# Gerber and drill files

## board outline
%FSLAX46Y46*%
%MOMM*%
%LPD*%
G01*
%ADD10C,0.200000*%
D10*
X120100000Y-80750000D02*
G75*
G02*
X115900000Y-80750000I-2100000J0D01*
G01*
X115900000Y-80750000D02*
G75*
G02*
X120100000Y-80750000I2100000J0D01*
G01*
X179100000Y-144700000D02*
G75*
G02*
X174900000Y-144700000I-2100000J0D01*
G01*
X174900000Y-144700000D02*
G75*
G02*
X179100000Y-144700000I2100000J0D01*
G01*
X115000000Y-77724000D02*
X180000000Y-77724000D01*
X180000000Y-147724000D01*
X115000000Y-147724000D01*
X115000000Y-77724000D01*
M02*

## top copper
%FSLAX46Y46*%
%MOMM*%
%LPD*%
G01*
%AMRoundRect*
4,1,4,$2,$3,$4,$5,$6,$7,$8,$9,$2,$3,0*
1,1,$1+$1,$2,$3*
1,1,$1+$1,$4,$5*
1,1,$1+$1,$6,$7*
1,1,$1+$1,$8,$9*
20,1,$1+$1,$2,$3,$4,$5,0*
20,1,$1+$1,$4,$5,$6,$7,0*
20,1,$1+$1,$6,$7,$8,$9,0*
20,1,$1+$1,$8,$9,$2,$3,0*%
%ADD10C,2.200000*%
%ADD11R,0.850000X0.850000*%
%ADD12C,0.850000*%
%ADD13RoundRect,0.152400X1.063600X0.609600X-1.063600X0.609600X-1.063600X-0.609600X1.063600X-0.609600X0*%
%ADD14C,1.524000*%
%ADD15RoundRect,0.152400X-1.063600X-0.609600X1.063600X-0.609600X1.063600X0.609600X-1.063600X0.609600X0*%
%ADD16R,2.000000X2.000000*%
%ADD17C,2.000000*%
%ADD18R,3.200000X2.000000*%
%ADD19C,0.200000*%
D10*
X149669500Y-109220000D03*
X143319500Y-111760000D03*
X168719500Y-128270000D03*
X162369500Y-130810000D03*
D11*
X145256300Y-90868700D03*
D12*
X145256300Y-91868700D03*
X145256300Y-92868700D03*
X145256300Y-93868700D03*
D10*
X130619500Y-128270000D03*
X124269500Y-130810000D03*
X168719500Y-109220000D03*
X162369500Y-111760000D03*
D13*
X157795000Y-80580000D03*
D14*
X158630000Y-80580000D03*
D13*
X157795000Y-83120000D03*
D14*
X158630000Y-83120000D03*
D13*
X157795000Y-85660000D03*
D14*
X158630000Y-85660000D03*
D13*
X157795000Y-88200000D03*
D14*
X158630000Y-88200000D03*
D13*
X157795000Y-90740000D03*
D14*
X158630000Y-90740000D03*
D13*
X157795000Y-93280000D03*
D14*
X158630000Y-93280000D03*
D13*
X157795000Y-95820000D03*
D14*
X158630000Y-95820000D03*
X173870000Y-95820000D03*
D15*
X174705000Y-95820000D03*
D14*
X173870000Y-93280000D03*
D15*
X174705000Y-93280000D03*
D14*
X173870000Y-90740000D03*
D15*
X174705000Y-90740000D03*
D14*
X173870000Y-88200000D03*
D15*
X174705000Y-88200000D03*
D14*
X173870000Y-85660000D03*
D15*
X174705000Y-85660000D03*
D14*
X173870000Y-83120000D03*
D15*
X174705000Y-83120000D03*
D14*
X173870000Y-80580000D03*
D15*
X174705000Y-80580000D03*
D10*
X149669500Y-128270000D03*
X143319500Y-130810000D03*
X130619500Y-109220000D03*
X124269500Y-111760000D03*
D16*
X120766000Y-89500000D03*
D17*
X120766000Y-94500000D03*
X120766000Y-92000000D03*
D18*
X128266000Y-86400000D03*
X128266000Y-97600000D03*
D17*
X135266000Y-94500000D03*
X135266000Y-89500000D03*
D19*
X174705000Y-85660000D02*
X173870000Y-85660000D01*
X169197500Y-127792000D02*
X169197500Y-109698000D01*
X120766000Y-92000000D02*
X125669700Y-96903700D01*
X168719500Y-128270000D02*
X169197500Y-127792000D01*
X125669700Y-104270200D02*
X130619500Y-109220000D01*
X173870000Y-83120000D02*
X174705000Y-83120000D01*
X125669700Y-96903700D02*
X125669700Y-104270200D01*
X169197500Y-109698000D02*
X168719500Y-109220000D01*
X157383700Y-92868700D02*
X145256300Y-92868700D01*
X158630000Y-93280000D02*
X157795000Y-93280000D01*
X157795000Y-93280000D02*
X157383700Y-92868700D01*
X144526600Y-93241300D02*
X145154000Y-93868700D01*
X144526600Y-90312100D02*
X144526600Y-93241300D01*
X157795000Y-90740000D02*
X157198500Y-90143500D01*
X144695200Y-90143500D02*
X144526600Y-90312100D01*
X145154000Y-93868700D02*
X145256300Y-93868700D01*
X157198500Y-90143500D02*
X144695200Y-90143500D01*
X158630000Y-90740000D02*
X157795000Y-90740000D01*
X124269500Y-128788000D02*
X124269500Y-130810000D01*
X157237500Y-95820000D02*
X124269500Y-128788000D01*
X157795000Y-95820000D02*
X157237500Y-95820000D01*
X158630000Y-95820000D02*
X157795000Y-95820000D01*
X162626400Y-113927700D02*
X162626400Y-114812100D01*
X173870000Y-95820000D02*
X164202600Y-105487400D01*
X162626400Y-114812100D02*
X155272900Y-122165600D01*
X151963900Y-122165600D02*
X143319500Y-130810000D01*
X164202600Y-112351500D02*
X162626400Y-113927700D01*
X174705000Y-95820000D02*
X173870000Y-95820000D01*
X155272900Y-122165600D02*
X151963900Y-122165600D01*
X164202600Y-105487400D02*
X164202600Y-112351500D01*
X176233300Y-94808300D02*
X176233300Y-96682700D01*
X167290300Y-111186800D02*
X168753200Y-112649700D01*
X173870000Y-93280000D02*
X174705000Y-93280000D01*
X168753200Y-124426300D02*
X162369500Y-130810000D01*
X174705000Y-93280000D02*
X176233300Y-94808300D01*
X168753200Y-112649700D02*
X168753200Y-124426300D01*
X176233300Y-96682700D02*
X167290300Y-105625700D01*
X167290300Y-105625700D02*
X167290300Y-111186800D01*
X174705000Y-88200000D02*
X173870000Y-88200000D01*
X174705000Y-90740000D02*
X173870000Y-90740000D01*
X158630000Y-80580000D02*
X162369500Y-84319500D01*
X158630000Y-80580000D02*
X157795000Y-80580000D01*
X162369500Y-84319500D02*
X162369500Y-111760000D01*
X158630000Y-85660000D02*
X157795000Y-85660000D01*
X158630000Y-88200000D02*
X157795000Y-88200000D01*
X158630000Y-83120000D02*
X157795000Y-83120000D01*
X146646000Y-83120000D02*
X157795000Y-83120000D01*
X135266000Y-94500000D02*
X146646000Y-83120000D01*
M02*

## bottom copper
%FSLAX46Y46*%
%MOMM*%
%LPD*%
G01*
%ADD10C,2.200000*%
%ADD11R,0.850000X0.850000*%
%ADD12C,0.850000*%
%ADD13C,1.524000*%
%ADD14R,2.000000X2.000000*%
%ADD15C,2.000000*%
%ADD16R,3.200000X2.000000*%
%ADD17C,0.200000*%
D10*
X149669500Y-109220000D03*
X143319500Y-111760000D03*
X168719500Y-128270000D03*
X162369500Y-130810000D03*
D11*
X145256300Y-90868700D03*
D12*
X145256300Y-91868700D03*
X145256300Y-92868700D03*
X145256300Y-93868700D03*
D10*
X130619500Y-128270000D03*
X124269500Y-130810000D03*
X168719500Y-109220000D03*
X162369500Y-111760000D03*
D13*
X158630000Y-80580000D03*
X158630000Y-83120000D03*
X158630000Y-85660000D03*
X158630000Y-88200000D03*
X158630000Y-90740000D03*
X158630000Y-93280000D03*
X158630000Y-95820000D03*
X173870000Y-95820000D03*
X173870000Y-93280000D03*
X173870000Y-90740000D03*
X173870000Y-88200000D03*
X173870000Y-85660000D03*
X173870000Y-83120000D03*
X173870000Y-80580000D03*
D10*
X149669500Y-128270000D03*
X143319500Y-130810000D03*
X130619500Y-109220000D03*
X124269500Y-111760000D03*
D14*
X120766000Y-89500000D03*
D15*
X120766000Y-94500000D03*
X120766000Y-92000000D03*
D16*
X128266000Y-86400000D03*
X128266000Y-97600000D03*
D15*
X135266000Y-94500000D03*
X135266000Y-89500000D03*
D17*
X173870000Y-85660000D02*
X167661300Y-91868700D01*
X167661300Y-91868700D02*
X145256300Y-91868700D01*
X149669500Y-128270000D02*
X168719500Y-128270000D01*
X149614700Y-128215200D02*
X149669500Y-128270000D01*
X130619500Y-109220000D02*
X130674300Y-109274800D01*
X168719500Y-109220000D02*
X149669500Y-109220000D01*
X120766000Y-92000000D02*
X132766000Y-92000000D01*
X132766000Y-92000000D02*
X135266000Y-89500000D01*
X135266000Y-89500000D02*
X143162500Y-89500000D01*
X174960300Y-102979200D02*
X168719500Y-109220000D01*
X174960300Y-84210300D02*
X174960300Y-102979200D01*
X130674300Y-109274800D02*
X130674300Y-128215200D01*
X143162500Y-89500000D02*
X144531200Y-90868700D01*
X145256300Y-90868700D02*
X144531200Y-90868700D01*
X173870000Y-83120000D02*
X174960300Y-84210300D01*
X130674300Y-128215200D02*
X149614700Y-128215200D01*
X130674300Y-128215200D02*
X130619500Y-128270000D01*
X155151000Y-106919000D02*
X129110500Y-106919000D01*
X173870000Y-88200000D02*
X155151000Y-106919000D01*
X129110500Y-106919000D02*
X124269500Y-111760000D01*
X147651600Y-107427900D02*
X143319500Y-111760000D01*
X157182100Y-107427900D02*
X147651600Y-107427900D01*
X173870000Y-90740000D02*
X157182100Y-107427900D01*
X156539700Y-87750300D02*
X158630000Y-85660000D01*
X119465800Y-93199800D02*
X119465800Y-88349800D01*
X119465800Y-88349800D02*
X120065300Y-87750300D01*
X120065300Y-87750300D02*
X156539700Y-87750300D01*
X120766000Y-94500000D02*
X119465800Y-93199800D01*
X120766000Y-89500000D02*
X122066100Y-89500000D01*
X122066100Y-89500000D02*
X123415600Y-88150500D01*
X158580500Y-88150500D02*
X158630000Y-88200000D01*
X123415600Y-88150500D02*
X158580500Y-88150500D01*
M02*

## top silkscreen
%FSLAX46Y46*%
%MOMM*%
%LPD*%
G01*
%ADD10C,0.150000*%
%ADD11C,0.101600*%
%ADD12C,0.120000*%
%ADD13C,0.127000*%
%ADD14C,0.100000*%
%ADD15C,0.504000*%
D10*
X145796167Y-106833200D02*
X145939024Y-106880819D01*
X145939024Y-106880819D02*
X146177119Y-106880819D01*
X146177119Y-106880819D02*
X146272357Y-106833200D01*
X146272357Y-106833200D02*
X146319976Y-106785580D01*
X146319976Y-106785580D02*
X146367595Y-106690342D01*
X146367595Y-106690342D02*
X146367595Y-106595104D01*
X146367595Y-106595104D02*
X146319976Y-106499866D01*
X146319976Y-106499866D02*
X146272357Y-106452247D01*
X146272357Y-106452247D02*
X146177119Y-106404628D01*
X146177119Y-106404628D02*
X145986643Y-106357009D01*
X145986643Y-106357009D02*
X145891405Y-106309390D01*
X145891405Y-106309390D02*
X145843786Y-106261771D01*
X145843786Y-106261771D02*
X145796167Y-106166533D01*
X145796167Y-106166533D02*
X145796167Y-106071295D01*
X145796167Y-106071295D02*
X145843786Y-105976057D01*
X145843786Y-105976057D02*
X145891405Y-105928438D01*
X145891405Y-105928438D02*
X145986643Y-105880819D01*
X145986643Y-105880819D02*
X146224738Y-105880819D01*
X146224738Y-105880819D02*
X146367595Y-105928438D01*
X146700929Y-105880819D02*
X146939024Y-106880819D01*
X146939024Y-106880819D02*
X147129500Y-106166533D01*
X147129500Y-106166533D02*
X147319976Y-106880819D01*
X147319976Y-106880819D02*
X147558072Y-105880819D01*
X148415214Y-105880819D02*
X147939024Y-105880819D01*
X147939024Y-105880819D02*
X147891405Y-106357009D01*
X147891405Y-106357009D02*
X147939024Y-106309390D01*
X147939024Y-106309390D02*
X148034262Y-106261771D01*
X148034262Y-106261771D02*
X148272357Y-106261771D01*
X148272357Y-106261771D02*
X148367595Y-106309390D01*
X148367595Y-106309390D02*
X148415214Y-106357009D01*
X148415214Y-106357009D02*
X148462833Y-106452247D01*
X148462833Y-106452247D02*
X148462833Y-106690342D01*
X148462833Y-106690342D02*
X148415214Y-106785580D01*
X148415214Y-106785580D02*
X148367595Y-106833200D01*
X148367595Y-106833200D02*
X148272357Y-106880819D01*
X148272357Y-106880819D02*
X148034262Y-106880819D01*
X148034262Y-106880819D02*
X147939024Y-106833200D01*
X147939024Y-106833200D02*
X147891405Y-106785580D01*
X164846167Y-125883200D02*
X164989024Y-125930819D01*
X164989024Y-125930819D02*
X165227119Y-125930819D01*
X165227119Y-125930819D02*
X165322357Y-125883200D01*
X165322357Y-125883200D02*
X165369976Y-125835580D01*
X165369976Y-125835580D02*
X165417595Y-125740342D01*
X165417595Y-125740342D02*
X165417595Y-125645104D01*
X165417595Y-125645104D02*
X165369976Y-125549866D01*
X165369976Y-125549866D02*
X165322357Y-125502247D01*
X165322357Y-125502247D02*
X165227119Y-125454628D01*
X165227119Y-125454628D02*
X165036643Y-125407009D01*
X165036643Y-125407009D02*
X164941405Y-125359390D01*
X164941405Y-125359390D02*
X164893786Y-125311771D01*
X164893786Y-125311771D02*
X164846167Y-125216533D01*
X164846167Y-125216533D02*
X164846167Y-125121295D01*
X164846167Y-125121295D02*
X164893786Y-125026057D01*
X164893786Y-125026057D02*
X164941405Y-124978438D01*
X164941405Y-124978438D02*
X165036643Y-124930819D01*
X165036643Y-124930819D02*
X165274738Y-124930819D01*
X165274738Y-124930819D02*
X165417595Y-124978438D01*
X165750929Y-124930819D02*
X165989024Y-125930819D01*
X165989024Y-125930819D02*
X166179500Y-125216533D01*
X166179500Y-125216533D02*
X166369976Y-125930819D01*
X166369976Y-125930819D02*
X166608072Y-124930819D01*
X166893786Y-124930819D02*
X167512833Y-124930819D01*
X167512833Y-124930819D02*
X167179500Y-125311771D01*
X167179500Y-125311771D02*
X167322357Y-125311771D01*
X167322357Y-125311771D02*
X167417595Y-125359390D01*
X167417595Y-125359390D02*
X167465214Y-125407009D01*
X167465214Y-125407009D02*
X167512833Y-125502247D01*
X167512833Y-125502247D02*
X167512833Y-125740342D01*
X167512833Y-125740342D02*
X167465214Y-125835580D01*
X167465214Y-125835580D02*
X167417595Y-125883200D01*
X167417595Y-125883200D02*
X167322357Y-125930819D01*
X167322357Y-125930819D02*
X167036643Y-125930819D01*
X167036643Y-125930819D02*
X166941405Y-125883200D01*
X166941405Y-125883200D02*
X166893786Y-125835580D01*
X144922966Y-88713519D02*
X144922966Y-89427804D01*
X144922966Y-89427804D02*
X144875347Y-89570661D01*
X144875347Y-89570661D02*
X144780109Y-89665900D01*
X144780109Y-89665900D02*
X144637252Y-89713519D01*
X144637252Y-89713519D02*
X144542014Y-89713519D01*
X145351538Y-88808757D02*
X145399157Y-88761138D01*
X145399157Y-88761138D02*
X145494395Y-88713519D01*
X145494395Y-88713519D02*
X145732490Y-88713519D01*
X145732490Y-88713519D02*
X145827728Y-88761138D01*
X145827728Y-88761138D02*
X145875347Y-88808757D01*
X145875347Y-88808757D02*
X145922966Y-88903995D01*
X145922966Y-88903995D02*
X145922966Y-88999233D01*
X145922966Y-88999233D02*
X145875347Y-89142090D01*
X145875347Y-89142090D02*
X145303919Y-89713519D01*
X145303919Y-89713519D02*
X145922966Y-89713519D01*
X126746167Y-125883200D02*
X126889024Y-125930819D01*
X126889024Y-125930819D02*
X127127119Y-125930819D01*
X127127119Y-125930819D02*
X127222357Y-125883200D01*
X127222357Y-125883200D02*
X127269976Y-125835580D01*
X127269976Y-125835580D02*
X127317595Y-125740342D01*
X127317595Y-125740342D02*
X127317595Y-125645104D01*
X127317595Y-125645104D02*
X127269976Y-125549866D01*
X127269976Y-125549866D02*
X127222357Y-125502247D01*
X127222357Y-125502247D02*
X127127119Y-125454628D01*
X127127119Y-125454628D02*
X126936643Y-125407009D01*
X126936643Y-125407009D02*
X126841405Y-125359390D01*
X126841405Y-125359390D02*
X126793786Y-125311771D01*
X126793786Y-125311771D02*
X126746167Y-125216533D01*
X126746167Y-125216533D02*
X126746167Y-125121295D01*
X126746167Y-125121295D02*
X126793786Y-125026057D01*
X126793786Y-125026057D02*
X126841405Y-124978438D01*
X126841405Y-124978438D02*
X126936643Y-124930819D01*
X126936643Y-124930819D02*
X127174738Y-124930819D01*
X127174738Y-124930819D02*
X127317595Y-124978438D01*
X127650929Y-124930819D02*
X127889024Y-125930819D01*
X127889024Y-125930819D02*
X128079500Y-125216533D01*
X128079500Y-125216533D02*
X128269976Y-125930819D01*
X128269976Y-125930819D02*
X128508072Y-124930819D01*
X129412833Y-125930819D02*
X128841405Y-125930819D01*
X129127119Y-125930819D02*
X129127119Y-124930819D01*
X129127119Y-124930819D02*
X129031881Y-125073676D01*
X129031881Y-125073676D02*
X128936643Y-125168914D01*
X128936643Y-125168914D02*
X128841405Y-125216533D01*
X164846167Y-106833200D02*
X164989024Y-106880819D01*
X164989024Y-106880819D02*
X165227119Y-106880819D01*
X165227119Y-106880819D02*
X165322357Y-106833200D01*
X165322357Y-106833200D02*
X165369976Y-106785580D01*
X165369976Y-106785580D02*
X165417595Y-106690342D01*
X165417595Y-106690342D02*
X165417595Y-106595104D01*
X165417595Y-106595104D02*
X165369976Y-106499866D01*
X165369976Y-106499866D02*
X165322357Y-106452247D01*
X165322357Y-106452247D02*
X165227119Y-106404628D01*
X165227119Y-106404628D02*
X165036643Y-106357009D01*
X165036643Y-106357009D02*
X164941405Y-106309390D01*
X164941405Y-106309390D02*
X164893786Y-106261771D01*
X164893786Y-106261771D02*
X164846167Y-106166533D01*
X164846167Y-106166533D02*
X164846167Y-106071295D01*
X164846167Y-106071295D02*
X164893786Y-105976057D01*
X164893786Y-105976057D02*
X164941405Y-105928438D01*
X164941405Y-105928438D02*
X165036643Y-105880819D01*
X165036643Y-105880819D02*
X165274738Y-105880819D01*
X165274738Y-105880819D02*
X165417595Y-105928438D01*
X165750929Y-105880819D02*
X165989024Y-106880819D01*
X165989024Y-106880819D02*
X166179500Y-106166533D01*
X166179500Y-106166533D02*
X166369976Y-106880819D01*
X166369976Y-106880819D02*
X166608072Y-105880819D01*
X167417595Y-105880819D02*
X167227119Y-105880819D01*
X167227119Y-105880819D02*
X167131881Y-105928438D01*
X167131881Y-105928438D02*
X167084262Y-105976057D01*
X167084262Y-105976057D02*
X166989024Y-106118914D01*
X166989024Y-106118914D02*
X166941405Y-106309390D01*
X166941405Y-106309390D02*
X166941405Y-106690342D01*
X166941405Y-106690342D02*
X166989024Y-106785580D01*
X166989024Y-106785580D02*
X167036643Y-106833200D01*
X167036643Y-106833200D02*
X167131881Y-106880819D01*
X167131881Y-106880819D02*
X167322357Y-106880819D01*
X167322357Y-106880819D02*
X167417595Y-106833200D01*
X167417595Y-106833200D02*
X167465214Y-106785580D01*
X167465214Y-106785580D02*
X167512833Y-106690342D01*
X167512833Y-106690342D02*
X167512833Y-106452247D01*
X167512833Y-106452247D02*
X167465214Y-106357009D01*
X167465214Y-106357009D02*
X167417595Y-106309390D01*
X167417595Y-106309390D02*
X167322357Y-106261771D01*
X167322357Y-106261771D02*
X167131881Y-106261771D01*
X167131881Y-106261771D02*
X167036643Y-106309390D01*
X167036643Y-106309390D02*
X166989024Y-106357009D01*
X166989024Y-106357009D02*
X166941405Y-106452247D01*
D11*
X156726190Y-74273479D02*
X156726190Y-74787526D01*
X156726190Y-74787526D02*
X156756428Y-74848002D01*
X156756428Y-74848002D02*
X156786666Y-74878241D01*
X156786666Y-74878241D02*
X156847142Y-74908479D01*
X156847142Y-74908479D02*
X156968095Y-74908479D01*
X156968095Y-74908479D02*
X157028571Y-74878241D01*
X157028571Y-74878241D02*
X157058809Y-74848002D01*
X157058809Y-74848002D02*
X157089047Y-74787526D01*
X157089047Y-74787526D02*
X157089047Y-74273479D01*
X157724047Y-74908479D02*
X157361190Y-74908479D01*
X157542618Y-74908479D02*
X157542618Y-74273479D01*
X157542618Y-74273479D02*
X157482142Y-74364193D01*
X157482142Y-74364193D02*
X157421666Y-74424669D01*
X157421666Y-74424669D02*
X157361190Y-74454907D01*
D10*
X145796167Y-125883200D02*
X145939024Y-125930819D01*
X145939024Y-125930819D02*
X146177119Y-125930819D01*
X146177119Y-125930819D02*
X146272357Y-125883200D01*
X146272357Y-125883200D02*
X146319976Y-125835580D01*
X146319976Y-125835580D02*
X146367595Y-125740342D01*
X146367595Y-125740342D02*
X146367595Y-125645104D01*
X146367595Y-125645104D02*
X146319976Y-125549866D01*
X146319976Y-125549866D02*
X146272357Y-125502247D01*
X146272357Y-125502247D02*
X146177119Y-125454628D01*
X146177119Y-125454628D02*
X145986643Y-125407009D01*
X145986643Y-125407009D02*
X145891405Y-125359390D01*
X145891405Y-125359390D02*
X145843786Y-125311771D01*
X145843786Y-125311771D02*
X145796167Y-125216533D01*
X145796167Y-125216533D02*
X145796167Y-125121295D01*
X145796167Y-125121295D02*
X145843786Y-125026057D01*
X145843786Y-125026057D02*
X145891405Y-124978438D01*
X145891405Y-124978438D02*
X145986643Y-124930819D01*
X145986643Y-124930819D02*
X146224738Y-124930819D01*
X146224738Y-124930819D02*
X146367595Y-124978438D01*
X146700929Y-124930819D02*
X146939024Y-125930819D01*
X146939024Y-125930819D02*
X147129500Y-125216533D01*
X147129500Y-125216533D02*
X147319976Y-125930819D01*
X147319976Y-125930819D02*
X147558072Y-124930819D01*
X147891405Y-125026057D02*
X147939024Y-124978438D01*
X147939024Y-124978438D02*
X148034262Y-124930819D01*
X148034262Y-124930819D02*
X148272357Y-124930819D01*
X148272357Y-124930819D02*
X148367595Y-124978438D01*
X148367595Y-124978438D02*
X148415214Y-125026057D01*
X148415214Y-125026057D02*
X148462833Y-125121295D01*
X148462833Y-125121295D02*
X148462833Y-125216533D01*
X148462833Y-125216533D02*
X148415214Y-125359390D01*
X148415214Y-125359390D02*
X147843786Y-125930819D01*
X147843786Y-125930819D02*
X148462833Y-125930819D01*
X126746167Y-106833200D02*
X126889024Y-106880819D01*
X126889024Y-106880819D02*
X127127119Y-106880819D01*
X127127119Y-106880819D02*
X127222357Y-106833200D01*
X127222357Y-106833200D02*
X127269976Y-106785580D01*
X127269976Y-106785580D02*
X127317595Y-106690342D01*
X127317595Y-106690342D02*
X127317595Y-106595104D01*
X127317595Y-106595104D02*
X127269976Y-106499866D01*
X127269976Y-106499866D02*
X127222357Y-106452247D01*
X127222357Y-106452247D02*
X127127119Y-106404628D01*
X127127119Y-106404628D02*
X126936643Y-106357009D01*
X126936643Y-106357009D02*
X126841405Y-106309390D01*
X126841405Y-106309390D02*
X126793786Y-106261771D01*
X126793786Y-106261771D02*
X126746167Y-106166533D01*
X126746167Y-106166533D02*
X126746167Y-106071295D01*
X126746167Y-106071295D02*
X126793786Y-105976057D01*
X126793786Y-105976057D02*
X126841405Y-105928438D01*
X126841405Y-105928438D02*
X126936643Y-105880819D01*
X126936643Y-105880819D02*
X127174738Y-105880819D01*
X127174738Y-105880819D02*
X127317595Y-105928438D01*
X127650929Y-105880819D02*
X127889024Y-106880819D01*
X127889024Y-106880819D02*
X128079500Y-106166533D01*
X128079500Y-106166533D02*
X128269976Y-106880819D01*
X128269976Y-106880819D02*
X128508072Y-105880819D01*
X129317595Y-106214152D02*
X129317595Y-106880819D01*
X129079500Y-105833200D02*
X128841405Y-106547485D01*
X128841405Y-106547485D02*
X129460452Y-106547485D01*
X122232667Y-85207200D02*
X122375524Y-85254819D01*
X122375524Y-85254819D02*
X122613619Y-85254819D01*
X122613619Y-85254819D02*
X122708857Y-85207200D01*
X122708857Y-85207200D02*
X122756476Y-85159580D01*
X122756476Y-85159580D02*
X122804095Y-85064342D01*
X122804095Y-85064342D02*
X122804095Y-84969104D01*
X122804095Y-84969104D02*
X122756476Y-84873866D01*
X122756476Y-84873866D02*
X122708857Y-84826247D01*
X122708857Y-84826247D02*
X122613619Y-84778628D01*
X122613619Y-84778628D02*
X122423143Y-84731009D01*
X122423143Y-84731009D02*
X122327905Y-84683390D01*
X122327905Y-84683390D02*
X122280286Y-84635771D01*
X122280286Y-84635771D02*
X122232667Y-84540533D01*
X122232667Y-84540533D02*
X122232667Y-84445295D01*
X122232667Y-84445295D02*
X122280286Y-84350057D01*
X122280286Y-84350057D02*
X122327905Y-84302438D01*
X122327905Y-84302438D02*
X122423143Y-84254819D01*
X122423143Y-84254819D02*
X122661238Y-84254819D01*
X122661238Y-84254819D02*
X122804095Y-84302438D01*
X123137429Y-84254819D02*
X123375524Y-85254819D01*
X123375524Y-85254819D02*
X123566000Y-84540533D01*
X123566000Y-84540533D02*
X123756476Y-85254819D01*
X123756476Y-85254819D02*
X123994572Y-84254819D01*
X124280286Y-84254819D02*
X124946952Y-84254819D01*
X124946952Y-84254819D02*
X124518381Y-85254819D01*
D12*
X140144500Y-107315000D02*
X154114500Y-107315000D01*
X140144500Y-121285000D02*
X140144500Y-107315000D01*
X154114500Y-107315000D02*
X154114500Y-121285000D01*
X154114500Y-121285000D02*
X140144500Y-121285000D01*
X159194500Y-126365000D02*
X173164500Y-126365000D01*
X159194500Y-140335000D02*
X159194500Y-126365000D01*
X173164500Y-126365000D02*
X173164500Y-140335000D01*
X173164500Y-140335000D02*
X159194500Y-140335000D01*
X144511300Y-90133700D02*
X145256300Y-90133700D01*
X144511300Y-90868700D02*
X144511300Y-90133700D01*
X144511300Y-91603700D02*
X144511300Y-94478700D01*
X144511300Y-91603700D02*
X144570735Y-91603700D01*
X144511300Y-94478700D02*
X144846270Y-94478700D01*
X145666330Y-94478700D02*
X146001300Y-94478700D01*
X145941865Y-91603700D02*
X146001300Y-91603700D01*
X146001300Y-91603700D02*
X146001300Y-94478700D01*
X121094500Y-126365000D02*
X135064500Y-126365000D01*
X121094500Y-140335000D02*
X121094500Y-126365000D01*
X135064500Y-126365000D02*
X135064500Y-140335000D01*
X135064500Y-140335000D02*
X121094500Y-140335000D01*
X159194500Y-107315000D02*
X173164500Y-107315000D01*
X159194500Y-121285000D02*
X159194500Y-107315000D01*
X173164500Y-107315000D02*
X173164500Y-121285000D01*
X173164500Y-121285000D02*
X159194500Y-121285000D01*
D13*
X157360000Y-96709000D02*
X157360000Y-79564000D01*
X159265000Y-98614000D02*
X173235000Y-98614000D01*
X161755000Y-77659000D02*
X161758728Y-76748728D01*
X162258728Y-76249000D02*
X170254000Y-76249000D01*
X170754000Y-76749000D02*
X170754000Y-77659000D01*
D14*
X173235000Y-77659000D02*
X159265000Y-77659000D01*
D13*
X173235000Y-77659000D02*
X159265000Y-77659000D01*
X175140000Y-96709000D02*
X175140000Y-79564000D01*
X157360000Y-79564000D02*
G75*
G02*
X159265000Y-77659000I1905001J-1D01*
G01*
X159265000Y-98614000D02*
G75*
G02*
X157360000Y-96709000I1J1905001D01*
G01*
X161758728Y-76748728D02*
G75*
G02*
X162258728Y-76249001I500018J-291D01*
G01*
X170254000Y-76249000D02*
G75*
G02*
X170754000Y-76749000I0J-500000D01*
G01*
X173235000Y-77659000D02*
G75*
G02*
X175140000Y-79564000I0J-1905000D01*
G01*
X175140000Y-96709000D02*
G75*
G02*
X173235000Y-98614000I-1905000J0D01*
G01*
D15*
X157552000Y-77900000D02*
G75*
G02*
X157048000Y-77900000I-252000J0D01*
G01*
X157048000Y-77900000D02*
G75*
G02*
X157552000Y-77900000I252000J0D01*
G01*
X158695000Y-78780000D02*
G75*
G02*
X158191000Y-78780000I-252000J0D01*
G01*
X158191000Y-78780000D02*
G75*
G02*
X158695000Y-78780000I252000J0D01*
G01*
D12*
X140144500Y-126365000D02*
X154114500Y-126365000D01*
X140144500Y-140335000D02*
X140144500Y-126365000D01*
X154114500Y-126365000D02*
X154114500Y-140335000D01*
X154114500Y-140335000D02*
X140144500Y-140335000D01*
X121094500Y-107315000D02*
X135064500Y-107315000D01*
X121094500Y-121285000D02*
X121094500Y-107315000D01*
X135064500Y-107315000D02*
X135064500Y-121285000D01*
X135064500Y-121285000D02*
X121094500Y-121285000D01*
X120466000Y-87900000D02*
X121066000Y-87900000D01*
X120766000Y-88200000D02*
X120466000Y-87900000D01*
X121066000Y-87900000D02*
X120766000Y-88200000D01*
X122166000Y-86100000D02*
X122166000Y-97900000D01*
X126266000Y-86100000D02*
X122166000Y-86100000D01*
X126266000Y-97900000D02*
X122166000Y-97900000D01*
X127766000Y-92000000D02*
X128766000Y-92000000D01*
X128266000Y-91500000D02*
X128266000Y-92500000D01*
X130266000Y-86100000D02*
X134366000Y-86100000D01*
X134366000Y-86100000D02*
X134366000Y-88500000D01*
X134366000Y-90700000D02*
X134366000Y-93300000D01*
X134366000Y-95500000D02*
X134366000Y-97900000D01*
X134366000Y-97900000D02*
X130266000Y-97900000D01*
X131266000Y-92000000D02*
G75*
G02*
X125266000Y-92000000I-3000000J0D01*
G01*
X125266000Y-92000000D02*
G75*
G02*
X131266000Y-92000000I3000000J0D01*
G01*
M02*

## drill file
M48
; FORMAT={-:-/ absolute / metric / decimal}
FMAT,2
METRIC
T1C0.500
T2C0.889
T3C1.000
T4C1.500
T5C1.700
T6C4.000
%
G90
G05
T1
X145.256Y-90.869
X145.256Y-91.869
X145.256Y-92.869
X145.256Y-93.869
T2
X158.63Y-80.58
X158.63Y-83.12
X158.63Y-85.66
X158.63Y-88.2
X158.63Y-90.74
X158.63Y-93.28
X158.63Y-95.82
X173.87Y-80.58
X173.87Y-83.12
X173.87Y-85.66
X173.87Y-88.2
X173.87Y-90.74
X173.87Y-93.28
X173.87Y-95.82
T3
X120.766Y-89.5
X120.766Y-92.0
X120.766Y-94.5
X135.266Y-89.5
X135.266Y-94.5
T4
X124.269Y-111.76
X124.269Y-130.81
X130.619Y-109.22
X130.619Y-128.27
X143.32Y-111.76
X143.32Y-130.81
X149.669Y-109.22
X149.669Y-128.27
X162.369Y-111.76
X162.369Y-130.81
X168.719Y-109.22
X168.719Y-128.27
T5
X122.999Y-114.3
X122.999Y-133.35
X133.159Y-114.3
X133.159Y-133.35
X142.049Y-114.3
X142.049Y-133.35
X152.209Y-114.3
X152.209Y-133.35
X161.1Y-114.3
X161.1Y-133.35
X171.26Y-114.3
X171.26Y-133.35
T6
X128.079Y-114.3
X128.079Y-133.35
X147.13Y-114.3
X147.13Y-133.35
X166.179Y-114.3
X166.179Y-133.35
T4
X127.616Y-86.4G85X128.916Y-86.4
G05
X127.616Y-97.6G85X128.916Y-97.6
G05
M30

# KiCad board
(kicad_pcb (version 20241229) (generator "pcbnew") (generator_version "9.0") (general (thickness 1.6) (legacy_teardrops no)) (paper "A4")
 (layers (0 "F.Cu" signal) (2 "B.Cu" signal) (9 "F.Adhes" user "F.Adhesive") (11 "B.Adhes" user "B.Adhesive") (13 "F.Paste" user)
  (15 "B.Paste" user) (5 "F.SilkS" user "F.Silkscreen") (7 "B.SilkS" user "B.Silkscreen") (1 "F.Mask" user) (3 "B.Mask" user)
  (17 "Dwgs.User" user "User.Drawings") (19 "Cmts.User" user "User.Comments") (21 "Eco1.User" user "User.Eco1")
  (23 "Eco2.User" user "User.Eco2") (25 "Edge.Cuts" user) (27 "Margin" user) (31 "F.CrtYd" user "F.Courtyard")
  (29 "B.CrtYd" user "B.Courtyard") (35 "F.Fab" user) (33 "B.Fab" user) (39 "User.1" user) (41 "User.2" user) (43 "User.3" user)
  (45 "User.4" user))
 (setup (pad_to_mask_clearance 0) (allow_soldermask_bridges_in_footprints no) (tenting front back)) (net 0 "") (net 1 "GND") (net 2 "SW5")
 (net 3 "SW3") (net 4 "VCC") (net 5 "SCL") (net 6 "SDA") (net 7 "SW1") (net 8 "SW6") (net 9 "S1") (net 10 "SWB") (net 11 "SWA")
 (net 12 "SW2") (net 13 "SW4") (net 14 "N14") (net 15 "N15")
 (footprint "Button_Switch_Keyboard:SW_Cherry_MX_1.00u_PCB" (layer "F.Cu") (at 149.6695 109.22)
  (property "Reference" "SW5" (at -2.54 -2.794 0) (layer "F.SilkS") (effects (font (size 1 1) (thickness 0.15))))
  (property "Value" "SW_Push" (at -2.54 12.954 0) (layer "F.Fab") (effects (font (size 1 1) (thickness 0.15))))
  (fp_line (start -9.525 -1.905) (end 4.445 -1.905) (stroke (width 0.12) (type solid)) (layer "F.SilkS"))
  (fp_line (start -9.525 12.065) (end -9.525 -1.905) (stroke (width 0.12) (type solid)) (layer "F.SilkS"))
  (fp_line (start 4.445 -1.905) (end 4.445 12.065) (stroke (width 0.12) (type solid)) (layer "F.SilkS"))
  (fp_line (start 4.445 12.065) (end -9.525 12.065) (stroke (width 0.12) (type solid)) (layer "F.SilkS"))
  (pad "" np_thru_hole circle (at -7.62 5.08) (size 1.7 1.7) (drill 1.7) (layers "*.Cu" "*.Mask"))
  (pad "" np_thru_hole circle (at -2.54 5.08) (size 4 4) (drill 4) (layers "*.Cu" "*.Mask"))
  (pad "" np_thru_hole circle (at 2.54 5.08) (size 1.7 1.7) (drill 1.7) (layers "*.Cu" "*.Mask"))
  (pad "1" thru_hole circle (at 0 0) (size 2.2 2.2) (drill 1.5) (layers "*.Cu" "*.Mask") (remove_unused_layers no) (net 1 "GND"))
  (pad "2" thru_hole circle (at -6.35 2.54) (size 2.2 2.2) (drill 1.5) (layers "*.Cu" "*.Mask") (remove_unused_layers no) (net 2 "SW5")))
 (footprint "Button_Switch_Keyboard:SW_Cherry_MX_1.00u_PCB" (layer "F.Cu") (at 168.7195 128.27)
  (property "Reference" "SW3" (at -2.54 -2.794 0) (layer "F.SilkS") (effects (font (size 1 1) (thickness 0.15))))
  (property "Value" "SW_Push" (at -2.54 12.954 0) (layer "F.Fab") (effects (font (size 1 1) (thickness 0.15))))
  (fp_line (start -9.525 -1.905) (end 4.445 -1.905) (stroke (width 0.12) (type solid)) (layer "F.SilkS"))
  (fp_line (start -9.525 12.065) (end -9.525 -1.905) (stroke (width 0.12) (type solid)) (layer "F.SilkS"))
  (fp_line (start 4.445 -1.905) (end 4.445 12.065) (stroke (width 0.12) (type solid)) (layer "F.SilkS"))
  (fp_line (start 4.445 12.065) (end -9.525 12.065) (stroke (width 0.12) (type solid)) (layer "F.SilkS"))
  (pad "" np_thru_hole circle (at -7.62 5.08) (size 1.7 1.7) (drill 1.7) (layers "*.Cu" "*.Mask"))
  (pad "" np_thru_hole circle (at -2.54 5.08) (size 4 4) (drill 4) (layers "*.Cu" "*.Mask"))
  (pad "" np_thru_hole circle (at 2.54 5.08) (size 1.7 1.7) (drill 1.7) (layers "*.Cu" "*.Mask"))
  (pad "1" thru_hole circle (at 0 0) (size 2.2 2.2) (drill 1.5) (layers "*.Cu" "*.Mask") (remove_unused_layers no) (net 1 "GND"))
  (pad "2" thru_hole circle (at -6.35 2.54) (size 2.2 2.2) (drill 1.5) (layers "*.Cu" "*.Mask") (remove_unused_layers no) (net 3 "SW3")))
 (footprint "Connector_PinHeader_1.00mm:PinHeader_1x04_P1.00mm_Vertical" (layer "F.Cu") (at 145.2563 90.8687)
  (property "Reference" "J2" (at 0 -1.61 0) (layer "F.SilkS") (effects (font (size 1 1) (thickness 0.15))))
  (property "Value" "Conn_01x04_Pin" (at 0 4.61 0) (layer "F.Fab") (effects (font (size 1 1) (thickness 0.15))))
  (fp_line (start -0.745 -0.735) (end 0 -0.735) (stroke (width 0.12) (type solid)) (layer "F.SilkS"))
  (fp_line (start -0.745 0) (end -0.745 -0.735) (stroke (width 0.12) (type solid)) (layer "F.SilkS"))
  (fp_line (start -0.745 0.735) (end -0.745 3.61) (stroke (width 0.12) (type solid)) (layer "F.SilkS"))
  (fp_line (start -0.745 0.735) (end -0.685565 0.735) (stroke (width 0.12) (type solid)) (layer "F.SilkS"))
  (fp_line (start -0.745 3.61) (end -0.41003 3.61) (stroke (width 0.12) (type solid)) (layer "F.SilkS"))
  (fp_line (start 0.41003 3.61) (end 0.745 3.61) (stroke (width 0.12) (type solid)) (layer "F.SilkS"))
  (fp_line (start 0.685565 0.735) (end 0.745 0.735) (stroke (width 0.12) (type solid)) (layer "F.SilkS"))
  (fp_line (start 0.745 0.735) (end 0.745 3.61) (stroke (width 0.12) (type solid)) (layer "F.SilkS"))
  (pad "1" thru_hole rect (at 0 0) (size 0.85 0.85) (drill 0.5) (layers "*.Cu" "*.Mask") (remove_unused_layers no) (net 1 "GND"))
  (pad "2" thru_hole circle (at 0 1) (size 0.85 0.85) (drill 0.5) (layers "*.Cu" "*.Mask") (remove_unused_layers no) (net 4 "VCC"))
  (pad "3" thru_hole circle (at 0 2) (size 0.85 0.85) (drill 0.5) (layers "*.Cu" "*.Mask") (remove_unused_layers no) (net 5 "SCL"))
  (pad "4" thru_hole circle (at 0 3) (size 0.85 0.85) (drill 0.5) (layers "*.Cu" "*.Mask") (remove_unused_layers no) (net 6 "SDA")))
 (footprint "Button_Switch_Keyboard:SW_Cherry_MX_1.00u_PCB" (layer "F.Cu") (at 130.6195 128.27)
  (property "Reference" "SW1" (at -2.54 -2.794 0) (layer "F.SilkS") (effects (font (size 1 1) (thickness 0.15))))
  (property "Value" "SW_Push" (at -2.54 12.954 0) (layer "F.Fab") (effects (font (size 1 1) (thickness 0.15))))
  (fp_line (start -9.525 -1.905) (end 4.445 -1.905) (stroke (width 0.12) (type solid)) (layer "F.SilkS"))
  (fp_line (start -9.525 12.065) (end -9.525 -1.905) (stroke (width 0.12) (type solid)) (layer "F.SilkS"))
  (fp_line (start 4.445 -1.905) (end 4.445 12.065) (stroke (width 0.12) (type solid)) (layer "F.SilkS"))
  (fp_line (start 4.445 12.065) (end -9.525 12.065) (stroke (width 0.12) (type solid)) (layer "F.SilkS"))
  (pad "" np_thru_hole circle (at -7.62 5.08) (size 1.7 1.7) (drill 1.7) (layers "*.Cu" "*.Mask"))
  (pad "" np_thru_hole circle (at -2.54 5.08) (size 4 4) (drill 4) (layers "*.Cu" "*.Mask"))
  (pad "" np_thru_hole circle (at 2.54 5.08) (size 1.7 1.7) (drill 1.7) (layers "*.Cu" "*.Mask"))
  (pad "1" thru_hole circle (at 0 0) (size 2.2 2.2) (drill 1.5) (layers "*.Cu" "*.Mask") (remove_unused_layers no) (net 1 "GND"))
  (pad "2" thru_hole circle (at -6.35 2.54) (size 2.2 2.2) (drill 1.5) (layers "*.Cu" "*.Mask") (remove_unused_layers no) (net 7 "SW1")))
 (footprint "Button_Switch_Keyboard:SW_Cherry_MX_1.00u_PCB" (layer "F.Cu") (at 168.7195 109.22)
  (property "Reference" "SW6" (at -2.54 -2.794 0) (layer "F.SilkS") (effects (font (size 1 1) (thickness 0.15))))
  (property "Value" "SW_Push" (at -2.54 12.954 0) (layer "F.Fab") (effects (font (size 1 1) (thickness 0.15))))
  (fp_line (start -9.525 -1.905) (end 4.445 -1.905) (stroke (width 0.12) (type solid)) (layer "F.SilkS"))
  (fp_line (start -9.525 12.065) (end -9.525 -1.905) (stroke (width 0.12) (type solid)) (layer "F.SilkS"))
  (fp_line (start 4.445 -1.905) (end 4.445 12.065) (stroke (width 0.12) (type solid)) (layer "F.SilkS"))
  (fp_line (start 4.445 12.065) (end -9.525 12.065) (stroke (width 0.12) (type solid)) (layer "F.SilkS"))
  (pad "" np_thru_hole circle (at -7.62 5.08) (size 1.7 1.7) (drill 1.7) (layers "*.Cu" "*.Mask"))
  (pad "" np_thru_hole circle (at -2.54 5.08) (size 4 4) (drill 4) (layers "*.Cu" "*.Mask"))
  (pad "" np_thru_hole circle (at 2.54 5.08) (size 1.7 1.7) (drill 1.7) (layers "*.Cu" "*.Mask"))
  (pad "1" thru_hole circle (at 0 0) (size 2.2 2.2) (drill 1.5) (layers "*.Cu" "*.Mask") (remove_unused_layers no) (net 1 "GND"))
  (pad "2" thru_hole circle (at -6.35 2.54) (size 2.2 2.2) (drill 1.5) (layers "*.Cu" "*.Mask") (remove_unused_layers no) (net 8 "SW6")))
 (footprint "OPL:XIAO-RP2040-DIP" (layer "F.Cu") (at 166.25 88.2)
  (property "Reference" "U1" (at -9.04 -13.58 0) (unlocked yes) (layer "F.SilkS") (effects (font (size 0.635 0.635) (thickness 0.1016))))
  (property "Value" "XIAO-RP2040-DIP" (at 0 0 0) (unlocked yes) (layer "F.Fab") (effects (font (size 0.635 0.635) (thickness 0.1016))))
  (fp_line (start -8.89 8.509) (end -8.89 -8.636) (stroke (width 0.127) (type solid)) (layer "F.SilkS"))
  (fp_line (start -6.985 10.414) (end 6.985 10.414) (stroke (width 0.127) (type solid)) (layer "F.SilkS"))
  (fp_line (start -4.495 -10.541) (end -4.491272 -11.451272) (stroke (width 0.127) (type solid)) (layer "F.SilkS"))
  (fp_line (start -3.991272 -11.951) (end 4.004 -11.951) (stroke (width 0.127) (type solid)) (layer "F.SilkS"))
  (fp_line (start 4.504 -11.451) (end 4.504 -10.541) (stroke (width 0.127) (type solid)) (layer "F.SilkS"))
  (fp_line (start 6.985 -10.541) (end -6.985 -10.541) (stroke (width 0.1) (type solid)) (layer "F.SilkS"))
  (fp_line (start 6.985 -10.541) (end -6.985 -10.541) (stroke (width 0.127) (type solid)) (layer "F.SilkS"))
  (fp_line (start 8.89 8.509) (end 8.89 -8.636) (stroke (width 0.127) (type solid)) (layer "F.SilkS"))
  (fp_arc (start -8.89 -8.636) (mid -8.332038 -9.983038) (end -6.985 -10.541) (stroke (width 0.127) (type solid)) (layer "F.SilkS"))
  (fp_arc (start -6.985 10.414) (mid -8.332038 9.856038) (end -8.89 8.509) (stroke (width 0.127) (type solid)) (layer "F.SilkS"))
  (fp_arc (start -4.491272 -11.451272) (mid -4.344728 -11.80464) (end -3.991272 -11.951) (stroke (width 0.127) (type default))
   (layer "F.SilkS"))
  (fp_arc (start 4.004 -11.951) (mid 4.357553 -11.804553) (end 4.504 -11.451) (stroke (width 0.127) (type default)) (layer "F.SilkS"))
  (fp_arc (start 6.985 -10.541) (mid 8.332038 -9.983038) (end 8.89 -8.636) (stroke (width 0.127) (type solid)) (layer "F.SilkS"))
  (fp_arc (start 8.89 8.509) (mid 8.332038 9.856038) (end 6.985 10.414) (stroke (width 0.127) (type solid)) (layer "F.SilkS"))
  (fp_circle (center -8.95 -10.3) (end -8.95 -10.554) (stroke (width 0.5) (type solid)) (fill yes) (layer "F.SilkS"))
  (fp_circle (center -7.807 -9.42) (end -7.807 -9.674) (stroke (width 0.5) (type solid)) (fill yes) (layer "F.SilkS"))
  (pad "1" smd roundrect (at -8.455 -7.62 180) (size 2.432 1.524) (layers "F.Cu" "F.Mask") (roundrect_rratio 0.1) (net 8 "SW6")
   (thermal_bridge_angle 45))
  (pad "1" thru_hole circle (at -7.62 -7.62 180) (size 1.524 1.524) (drill 0.889) (layers "*.Cu" "*.Mask") (remove_unused_layers no)
   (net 8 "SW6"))
  (pad "2" smd roundrect (at -8.455 -5.08 180) (size 2.432 1.524) (layers "F.Cu" "F.Mask") (roundrect_rratio 0.1) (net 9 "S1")
   (thermal_bridge_angle 45))
  (pad "2" thru_hole circle (at -7.62 -5.08 180) (size 1.524 1.524) (drill 0.889) (layers "*.Cu" "*.Mask") (remove_unused_layers no)
   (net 9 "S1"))
  (pad "3" smd roundrect (at -8.455 -2.54 180) (size 2.432 1.524) (layers "F.Cu" "F.Mask") (roundrect_rratio 0.1) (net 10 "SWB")
   (thermal_bridge_angle 45))
  (pad "3" thru_hole circle (at -7.62 -2.54 180) (size 1.524 1.524) (drill 0.889) (layers "*.Cu" "*.Mask") (remove_unused_layers no)
   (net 10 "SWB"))
  (pad "4" smd roundrect (at -8.455 0 180) (size 2.432 1.524) (layers "F.Cu" "F.Mask") (roundrect_rratio 0.1) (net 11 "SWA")
   (thermal_bridge_angle 45))
  (pad "4" thru_hole circle (at -7.62 0 180) (size 1.524 1.524) (drill 0.889) (layers "*.Cu" "*.Mask") (remove_unused_layers no)
   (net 11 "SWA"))
  (pad "5" smd roundrect (at -8.455 2.54 180) (size 2.432 1.524) (layers "F.Cu" "F.Mask") (roundrect_rratio 0.1) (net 6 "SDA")
   (thermal_bridge_angle 45))
  (pad "5" thru_hole circle (at -7.62 2.54 180) (size 1.524 1.524) (drill 0.889) (layers "*.Cu" "*.Mask") (remove_unused_layers no)
   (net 6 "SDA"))
  (pad "6" smd roundrect (at -8.455 5.08 180) (size 2.432 1.524) (layers "F.Cu" "F.Mask") (roundrect_rratio 0.1) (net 5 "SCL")
   (thermal_bridge_angle 45))
  (pad "6" thru_hole circle (at -7.62 5.08 180) (size 1.524 1.524) (drill 0.889) (layers "*.Cu" "*.Mask") (remove_unused_layers no)
   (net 5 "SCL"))
  (pad "7" smd roundrect (at -8.455 7.62 180) (size 2.432 1.524) (layers "F.Cu" "F.Mask") (roundrect_rratio 0.1) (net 7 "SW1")
   (thermal_bridge_angle 45))
  (pad "7" thru_hole circle (at -7.62 7.62 180) (size 1.524 1.524) (drill 0.889) (layers "*.Cu" "*.Mask") (remove_unused_layers no)
   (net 7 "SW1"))
  (pad "8" thru_hole circle (at 7.62 7.62) (size 1.524 1.524) (drill 0.889) (layers "*.Cu" "*.Mask") (remove_unused_layers no)
   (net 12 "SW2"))
  (pad "8" smd roundrect (at 8.455 7.62) (size 2.432 1.524) (layers "F.Cu" "F.Mask") (roundrect_rratio 0.1) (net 12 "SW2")
   (thermal_bridge_angle 45))
  (pad "9" thru_hole circle (at 7.62 5.08) (size 1.524 1.524) (drill 0.889) (layers "*.Cu" "*.Mask") (remove_unused_layers no) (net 3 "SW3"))
  (pad "9" smd roundrect (at 8.455 5.08) (size 2.432 1.524) (layers "F.Cu" "F.Mask") (roundrect_rratio 0.1) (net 3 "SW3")
   (thermal_bridge_angle 45))
  (pad "10" thru_hole circle (at 7.62 2.54) (size 1.524 1.524) (drill 0.889) (layers "*.Cu" "*.Mask") (remove_unused_layers no)
   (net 2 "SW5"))
  (pad "10" smd roundrect (at 8.455 2.54) (size 2.432 1.524) (layers "F.Cu" "F.Mask") (roundrect_rratio 0.1) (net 2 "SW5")
   (thermal_bridge_angle 45))
  (pad "11" thru_hole circle (at 7.62 0) (size 1.524 1.524) (drill 0.889) (layers "*.Cu" "*.Mask") (remove_unused_layers no) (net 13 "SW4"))
  (pad "11" smd roundrect (at 8.455 0) (size 2.432 1.524) (layers "F.Cu" "F.Mask") (roundrect_rratio 0.1) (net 13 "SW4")
   (thermal_bridge_angle 45))
  (pad "12" thru_hole circle (at 7.62 -2.54) (size 1.524 1.524) (drill 0.889) (layers "*.Cu" "*.Mask") (remove_unused_layers no)
   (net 4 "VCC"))
  (pad "12" smd roundrect (at 8.455 -2.54) (size 2.432 1.524) (layers "F.Cu" "F.Mask") (roundrect_rratio 0.1) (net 4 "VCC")
   (thermal_bridge_angle 45))
  (pad "13" thru_hole circle (at 7.62 -5.08) (size 1.524 1.524) (drill 0.889) (layers "*.Cu" "*.Mask") (remove_unused_layers no)
   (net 1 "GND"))
  (pad "13" smd roundrect (at 8.455 -5.08) (size 2.432 1.524) (layers "F.Cu" "F.Mask") (roundrect_rratio 0.1) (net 1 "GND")
   (thermal_bridge_angle 45))
  (pad "14" thru_hole circle (at 7.62 -7.62) (size 1.524 1.524) (drill 0.889) (layers "*.Cu" "*.Mask") (remove_unused_layers no)
   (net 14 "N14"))
  (pad "14" smd roundrect (at 8.455 -7.62) (size 2.432 1.524) (layers "F.Cu" "F.Mask") (roundrect_rratio 0.1) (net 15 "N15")
   (thermal_bridge_angle 45)))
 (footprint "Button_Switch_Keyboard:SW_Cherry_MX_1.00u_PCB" (layer "F.Cu") (at 149.6695 128.27)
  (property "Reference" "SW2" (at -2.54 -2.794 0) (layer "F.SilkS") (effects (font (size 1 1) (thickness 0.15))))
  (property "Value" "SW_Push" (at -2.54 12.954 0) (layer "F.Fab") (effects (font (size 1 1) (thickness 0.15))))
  (fp_line (start -9.525 -1.905) (end 4.445 -1.905) (stroke (width 0.12) (type solid)) (layer "F.SilkS"))
  (fp_line (start -9.525 12.065) (end -9.525 -1.905) (stroke (width 0.12) (type solid)) (layer "F.SilkS"))
  (fp_line (start 4.445 -1.905) (end 4.445 12.065) (stroke (width 0.12) (type solid)) (layer "F.SilkS"))
  (fp_line (start 4.445 12.065) (end -9.525 12.065) (stroke (width 0.12) (type solid)) (layer "F.SilkS"))
  (pad "" np_thru_hole circle (at -7.62 5.08) (size 1.7 1.7) (drill 1.7) (layers "*.Cu" "*.Mask"))
  (pad "" np_thru_hole circle (at -2.54 5.08) (size 4 4) (drill 4) (layers "*.Cu" "*.Mask"))
  (pad "" np_thru_hole circle (at 2.54 5.08) (size 1.7 1.7) (drill 1.7) (layers "*.Cu" "*.Mask"))
  (pad "1" thru_hole circle (at 0 0) (size 2.2 2.2) (drill 1.5) (layers "*.Cu" "*.Mask") (remove_unused_layers no) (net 1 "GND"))
  (pad "2" thru_hole circle (at -6.35 2.54) (size 2.2 2.2) (drill 1.5) (layers "*.Cu" "*.Mask") (remove_unused_layers no) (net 12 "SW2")))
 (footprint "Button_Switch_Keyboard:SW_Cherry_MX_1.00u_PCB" (layer "F.Cu") (at 130.6195 109.22)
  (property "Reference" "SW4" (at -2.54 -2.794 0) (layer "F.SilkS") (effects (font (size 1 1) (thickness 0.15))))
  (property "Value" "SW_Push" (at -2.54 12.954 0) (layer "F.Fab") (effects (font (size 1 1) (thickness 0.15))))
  (fp_line (start -9.525 -1.905) (end 4.445 -1.905) (stroke (width 0.12) (type solid)) (layer "F.SilkS"))
  (fp_line (start -9.525 12.065) (end -9.525 -1.905) (stroke (width 0.12) (type solid)) (layer "F.SilkS"))
  (fp_line (start 4.445 -1.905) (end 4.445 12.065) (stroke (width 0.12) (type solid)) (layer "F.SilkS"))
  (fp_line (start 4.445 12.065) (end -9.525 12.065) (stroke (width 0.12) (type solid)) (layer "F.SilkS"))
  (pad "" np_thru_hole circle (at -7.62 5.08) (size 1.7 1.7) (drill 1.7) (layers "*.Cu" "*.Mask"))
  (pad "" np_thru_hole circle (at -2.54 5.08) (size 4 4) (drill 4) (layers "*.Cu" "*.Mask"))
  (pad "" np_thru_hole circle (at 2.54 5.08) (size 1.7 1.7) (drill 1.7) (layers "*.Cu" "*.Mask"))
  (pad "1" thru_hole circle (at 0 0) (size 2.2 2.2) (drill 1.5) (layers "*.Cu" "*.Mask") (remove_unused_layers no) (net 1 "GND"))
  (pad "2" thru_hole circle (at -6.35 2.54) (size 2.2 2.2) (drill 1.5) (layers "*.Cu" "*.Mask") (remove_unused_layers no) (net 13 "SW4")))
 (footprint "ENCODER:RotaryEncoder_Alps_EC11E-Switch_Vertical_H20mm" (layer "F.Cu") (at 120.766 89.5)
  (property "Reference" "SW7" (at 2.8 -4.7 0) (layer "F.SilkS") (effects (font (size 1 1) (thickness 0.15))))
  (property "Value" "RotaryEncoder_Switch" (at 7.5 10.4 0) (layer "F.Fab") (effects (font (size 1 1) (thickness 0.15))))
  (fp_line (start -0.3 -1.6) (end 0.3 -1.6) (stroke (width 0.12) (type solid)) (layer "F.SilkS"))
  (fp_line (start 0 -1.3) (end -0.3 -1.6) (stroke (width 0.12) (type solid)) (layer "F.SilkS"))
  (fp_line (start 0.3 -1.6) (end 0 -1.3) (stroke (width 0.12) (type solid)) (layer "F.SilkS"))
  (fp_line (start 1.4 -3.4) (end 1.4 8.4) (stroke (width 0.12) (type solid)) (layer "F.SilkS"))
  (fp_line (start 5.5 -3.4) (end 1.4 -3.4) (stroke (width 0.12) (type solid)) (layer "F.SilkS"))
  (fp_line (start 5.5 8.4) (end 1.4 8.4) (stroke (width 0.12) (type solid)) (layer "F.SilkS"))
  (fp_line (start 7 2.5) (end 8 2.5) (stroke (width 0.12) (type solid)) (layer "F.SilkS"))
  (fp_line (start 7.5 2) (end 7.5 3) (stroke (width 0.12) (type solid)) (layer "F.SilkS"))
  (fp_line (start 9.5 -3.4) (end 13.6 -3.4) (stroke (width 0.12) (type solid)) (layer "F.SilkS"))
  (fp_line (start 13.6 -3.4) (end 13.6 -1) (stroke (width 0.12) (type solid)) (layer "F.SilkS"))
  (fp_line (start 13.6 1.2) (end 13.6 3.8) (stroke (width 0.12) (type solid)) (layer "F.SilkS"))
  (fp_line (start 13.6 6) (end 13.6 8.4) (stroke (width 0.12) (type solid)) (layer "F.SilkS"))
  (fp_line (start 13.6 8.4) (end 9.5 8.4) (stroke (width 0.12) (type solid)) (layer "F.SilkS"))
  (fp_circle (center 7.5 2.5) (end 10.5 2.5) (stroke (width 0.12) (type solid)) (fill no) (layer "F.SilkS"))
  (pad "A" thru_hole rect (at 0 0) (size 2 2) (drill 1) (layers "*.Cu" "*.Mask") (remove_unused_layers no) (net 11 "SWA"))
  (pad "B" thru_hole circle (at 0 5) (size 2 2) (drill 1) (layers "*.Cu" "*.Mask") (remove_unused_layers no) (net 10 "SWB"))
  (pad "C" thru_hole circle (at 0 2.5) (size 2 2) (drill 1) (layers "*.Cu" "*.Mask") (remove_unused_layers no) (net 1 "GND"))
  (pad "MP" thru_hole rect (at 7.5 -3.1) (size 3.2 2) (drill oval 2.8 1.5) (layers "*.Cu" "*.Mask") (remove_unused_layers no))
  (pad "MP" thru_hole rect (at 7.5 8.1) (size 3.2 2) (drill oval 2.8 1.5) (layers "*.Cu" "*.Mask") (remove_unused_layers no))
  (pad "S1" thru_hole circle (at 14.5 5) (size 2 2) (drill 1) (layers "*.Cu" "*.Mask") (remove_unused_layers no) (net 9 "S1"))
  (pad "S2" thru_hole circle (at 14.5 0) (size 2 2) (drill 1) (layers "*.Cu" "*.Mask") (remove_unused_layers no) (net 1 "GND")))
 (gr_circle (center 118 80.75) (end 120.1 80.75) (stroke (width 0.2) (type solid)) (fill no) (layer "Edge.Cuts"))
 (gr_circle (center 177 144.7) (end 179.1 144.7) (stroke (width 0.2) (type solid)) (fill no) (layer "Edge.Cuts"))
 (gr_rect (start 115 77.724) (end 180 147.724) (stroke (width 0.2) (type solid)) (fill no) (layer "Edge.Cuts"))
 (segment (start 174.705 85.66) (end 173.87 85.66) (width 0.2) (layer "F.Cu") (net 4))
 (segment (start 173.87 85.66) (end 167.6613 91.8687) (width 0.2) (layer "B.Cu") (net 4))
 (segment (start 167.6613 91.8687) (end 145.2563 91.8687) (width 0.2) (layer "B.Cu") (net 4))
 (segment (start 169.1975 127.792) (end 169.1975 109.698) (width 0.2) (layer "F.Cu") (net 1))
 (segment (start 120.766 92) (end 125.6697 96.9037) (width 0.2) (layer "F.Cu") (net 1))
 (segment (start 168.7195 128.27) (end 169.1975 127.792) (width 0.2) (layer "F.Cu") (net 1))
 (segment (start 125.6697 104.2702) (end 130.6195 109.22) (width 0.2) (layer "F.Cu") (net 1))
 (segment (start 173.87 83.12) (end 174.705 83.12) (width 0.2) (layer "F.Cu") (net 1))
 (segment (start 125.6697 96.9037) (end 125.6697 104.2702) (width 0.2) (layer "F.Cu") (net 1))
 (segment (start 169.1975 109.698) (end 168.7195 109.22) (width 0.2) (layer "F.Cu") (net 1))
 (segment (start 149.6695 128.27) (end 168.7195 128.27) (width 0.2) (layer "B.Cu") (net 1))
 (segment (start 149.6147 128.2152) (end 149.6695 128.27) (width 0.2) (layer "B.Cu") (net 1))
 (segment (start 130.6195 109.22) (end 130.6743 109.2748) (width 0.2) (layer "B.Cu") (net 1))
 (segment (start 168.7195 109.22) (end 149.6695 109.22) (width 0.2) (layer "B.Cu") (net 1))
 (segment (start 120.766 92) (end 132.766 92) (width 0.2) (layer "B.Cu") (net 1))
 (segment (start 132.766 92) (end 135.266 89.5) (width 0.2) (layer "B.Cu") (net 1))
 (segment (start 135.266 89.5) (end 143.1625 89.5) (width 0.2) (layer "B.Cu") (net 1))
 (segment (start 174.9603 102.9792) (end 168.7195 109.22) (width 0.2) (layer "B.Cu") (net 1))
 (segment (start 174.9603 84.2103) (end 174.9603 102.9792) (width 0.2) (layer "B.Cu") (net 1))
 (segment (start 130.6743 109.2748) (end 130.6743 128.2152) (width 0.2) (layer "B.Cu") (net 1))
 (segment (start 143.1625 89.5) (end 144.5312 90.8687) (width 0.2) (layer "B.Cu") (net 1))
 (segment (start 145.2563 90.8687) (end 144.5312 90.8687) (width 0.2) (layer "B.Cu") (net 1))
 (segment (start 173.87 83.12) (end 174.9603 84.2103) (width 0.2) (layer "B.Cu") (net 1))
 (segment (start 130.6743 128.2152) (end 149.6147 128.2152) (width 0.2) (layer "B.Cu") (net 1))
 (segment (start 130.6743 128.2152) (end 130.6195 128.27) (width 0.2) (layer "B.Cu") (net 1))
 (segment (start 157.3837 92.8687) (end 145.2563 92.8687) (width 0.2) (layer "F.Cu") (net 5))
 (segment (start 158.63 93.28) (end 157.795 93.28) (width 0.2) (layer "F.Cu") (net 5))
 (segment (start 157.795 93.28) (end 157.3837 92.8687) (width 0.2) (layer "F.Cu") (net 5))
 (segment (start 144.5266 93.2413) (end 145.154 93.8687) (width 0.2) (layer "F.Cu") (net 6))
 (segment (start 144.5266 90.3121) (end 144.5266 93.2413) (width 0.2) (layer "F.Cu") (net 6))
 (segment (start 157.795 90.74) (end 157.1985 90.1435) (width 0.2) (layer "F.Cu") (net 6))
 (segment (start 144.6952 90.1435) (end 144.5266 90.3121) (width 0.2) (layer "F.Cu") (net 6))
 (segment (start 145.154 93.8687) (end 145.2563 93.8687) (width 0.2) (layer "F.Cu") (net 6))
 (segment (start 157.1985 90.1435) (end 144.6952 90.1435) (width 0.2) (layer "F.Cu") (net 6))
 (segment (start 158.63 90.74) (end 157.795 90.74) (width 0.2) (layer "F.Cu") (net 6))
 (segment (start 124.2695 128.788) (end 124.2695 130.81) (width 0.2) (layer "F.Cu") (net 7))
 (segment (start 157.2375 95.82) (end 124.2695 128.788) (width 0.2) (layer "F.Cu") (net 7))
 (segment (start 157.795 95.82) (end 157.2375 95.82) (width 0.2) (layer "F.Cu") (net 7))
 (segment (start 158.63 95.82) (end 157.795 95.82) (width 0.2) (layer "F.Cu") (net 7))
 (segment (start 162.6264 113.9277) (end 162.6264 114.8121) (width 0.2) (layer "F.Cu") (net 12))
 (segment (start 173.87 95.82) (end 164.2026 105.4874) (width 0.2) (layer "F.Cu") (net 12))
 (segment (start 162.6264 114.8121) (end 155.2729 122.1656) (width 0.2) (layer "F.Cu") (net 12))
 (segment (start 151.9639 122.1656) (end 143.3195 130.81) (width 0.2) (layer "F.Cu") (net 12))
 (segment (start 164.2026 112.3515) (end 162.6264 113.9277) (width 0.2) (layer "F.Cu") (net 12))
 (segment (start 174.705 95.82) (end 173.87 95.82) (width 0.2) (layer "F.Cu") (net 12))
 (segment (start 155.2729 122.1656) (end 151.9639 122.1656) (width 0.2) (layer "F.Cu") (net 12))
 (segment (start 164.2026 105.4874) (end 164.2026 112.3515) (width 0.2) (layer "F.Cu") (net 12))
 (segment (start 176.2333 94.8083) (end 176.2333 96.6827) (width 0.2) (layer "F.Cu") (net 3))
 (segment (start 167.2903 111.1868) (end 168.7532 112.6497) (width 0.2) (layer "F.Cu") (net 3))
 (segment (start 173.87 93.28) (end 174.705 93.28) (width 0.2) (layer "F.Cu") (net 3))
 (segment (start 168.7532 124.4263) (end 162.3695 130.81) (width 0.2) (layer "F.Cu") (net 3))
 (segment (start 174.705 93.28) (end 176.2333 94.8083) (width 0.2) (layer "F.Cu") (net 3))
 (segment (start 168.7532 112.6497) (end 168.7532 124.4263) (width 0.2) (layer "F.Cu") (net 3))
 (segment (start 176.2333 96.6827) (end 167.2903 105.6257) (width 0.2) (layer "F.Cu") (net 3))
 (segment (start 167.2903 105.6257) (end 167.2903 111.1868) (width 0.2) (layer "F.Cu") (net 3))
 (segment (start 174.705 88.2) (end 173.87 88.2) (width 0.2) (layer "F.Cu") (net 13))
 (segment (start 155.151 106.919) (end 129.1105 106.919) (width 0.2) (layer "B.Cu") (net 13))
 (segment (start 173.87 88.2) (end 155.151 106.919) (width 0.2) (layer "B.Cu") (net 13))
 (segment (start 129.1105 106.919) (end 124.2695 111.76) (width 0.2) (layer "B.Cu") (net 13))
 (segment (start 174.705 90.74) (end 173.87 90.74) (width 0.2) (layer "F.Cu") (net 2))
 (segment (start 147.6516 107.4279) (end 143.3195 111.76) (width 0.2) (layer "B.Cu") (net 2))
 (segment (start 157.1821 107.4279) (end 147.6516 107.4279) (width 0.2) (layer "B.Cu") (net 2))
 (segment (start 173.87 90.74) (end 157.1821 107.4279) (width 0.2) (layer "B.Cu") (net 2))
 (segment (start 158.63 80.58) (end 162.3695 84.3195) (width 0.2) (layer "F.Cu") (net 8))
 (segment (start 158.63 80.58) (end 157.795 80.58) (width 0.2) (layer "F.Cu") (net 8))
 (segment (start 162.3695 84.3195) (end 162.3695 111.76) (width 0.2) (layer "F.Cu") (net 8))
 (segment (start 158.63 85.66) (end 157.795 85.66) (width 0.2) (layer "F.Cu") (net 10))
 (segment (start 156.5397 87.7503) (end 158.63 85.66) (width 0.2) (layer "B.Cu") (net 10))
 (segment (start 119.4658 93.1998) (end 119.4658 88.3498) (width 0.2) (layer "B.Cu") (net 10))
 (segment (start 119.4658 88.3498) (end 120.0653 87.7503) (width 0.2) (layer "B.Cu") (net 10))
 (segment (start 120.0653 87.7503) (end 156.5397 87.7503) (width 0.2) (layer "B.Cu") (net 10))
 (segment (start 120.766 94.5) (end 119.4658 93.1998) (width 0.2) (layer "B.Cu") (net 10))
 (segment (start 158.63 88.2) (end 157.795 88.2) (width 0.2) (layer "F.Cu") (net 11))
 (segment (start 120.766 89.5) (end 122.0661 89.5) (width 0.2) (layer "B.Cu") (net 11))
 (segment (start 122.0661 89.5) (end 123.4156 88.1505) (width 0.2) (layer "B.Cu") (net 11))
 (segment (start 158.5805 88.1505) (end 158.63 88.2) (width 0.2) (layer "B.Cu") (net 11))
 (segment (start 123.4156 88.1505) (end 158.5805 88.1505) (width 0.2) (layer "B.Cu") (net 11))
 (segment (start 158.63 83.12) (end 157.795 83.12) (width 0.2) (layer "F.Cu") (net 9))
 (segment (start 146.646 83.12) (end 157.795 83.12) (width 0.2) (layer "F.Cu") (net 9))
 (segment (start 135.266 94.5) (end 146.646 83.12) (width 0.2) (layer "F.Cu") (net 9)))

